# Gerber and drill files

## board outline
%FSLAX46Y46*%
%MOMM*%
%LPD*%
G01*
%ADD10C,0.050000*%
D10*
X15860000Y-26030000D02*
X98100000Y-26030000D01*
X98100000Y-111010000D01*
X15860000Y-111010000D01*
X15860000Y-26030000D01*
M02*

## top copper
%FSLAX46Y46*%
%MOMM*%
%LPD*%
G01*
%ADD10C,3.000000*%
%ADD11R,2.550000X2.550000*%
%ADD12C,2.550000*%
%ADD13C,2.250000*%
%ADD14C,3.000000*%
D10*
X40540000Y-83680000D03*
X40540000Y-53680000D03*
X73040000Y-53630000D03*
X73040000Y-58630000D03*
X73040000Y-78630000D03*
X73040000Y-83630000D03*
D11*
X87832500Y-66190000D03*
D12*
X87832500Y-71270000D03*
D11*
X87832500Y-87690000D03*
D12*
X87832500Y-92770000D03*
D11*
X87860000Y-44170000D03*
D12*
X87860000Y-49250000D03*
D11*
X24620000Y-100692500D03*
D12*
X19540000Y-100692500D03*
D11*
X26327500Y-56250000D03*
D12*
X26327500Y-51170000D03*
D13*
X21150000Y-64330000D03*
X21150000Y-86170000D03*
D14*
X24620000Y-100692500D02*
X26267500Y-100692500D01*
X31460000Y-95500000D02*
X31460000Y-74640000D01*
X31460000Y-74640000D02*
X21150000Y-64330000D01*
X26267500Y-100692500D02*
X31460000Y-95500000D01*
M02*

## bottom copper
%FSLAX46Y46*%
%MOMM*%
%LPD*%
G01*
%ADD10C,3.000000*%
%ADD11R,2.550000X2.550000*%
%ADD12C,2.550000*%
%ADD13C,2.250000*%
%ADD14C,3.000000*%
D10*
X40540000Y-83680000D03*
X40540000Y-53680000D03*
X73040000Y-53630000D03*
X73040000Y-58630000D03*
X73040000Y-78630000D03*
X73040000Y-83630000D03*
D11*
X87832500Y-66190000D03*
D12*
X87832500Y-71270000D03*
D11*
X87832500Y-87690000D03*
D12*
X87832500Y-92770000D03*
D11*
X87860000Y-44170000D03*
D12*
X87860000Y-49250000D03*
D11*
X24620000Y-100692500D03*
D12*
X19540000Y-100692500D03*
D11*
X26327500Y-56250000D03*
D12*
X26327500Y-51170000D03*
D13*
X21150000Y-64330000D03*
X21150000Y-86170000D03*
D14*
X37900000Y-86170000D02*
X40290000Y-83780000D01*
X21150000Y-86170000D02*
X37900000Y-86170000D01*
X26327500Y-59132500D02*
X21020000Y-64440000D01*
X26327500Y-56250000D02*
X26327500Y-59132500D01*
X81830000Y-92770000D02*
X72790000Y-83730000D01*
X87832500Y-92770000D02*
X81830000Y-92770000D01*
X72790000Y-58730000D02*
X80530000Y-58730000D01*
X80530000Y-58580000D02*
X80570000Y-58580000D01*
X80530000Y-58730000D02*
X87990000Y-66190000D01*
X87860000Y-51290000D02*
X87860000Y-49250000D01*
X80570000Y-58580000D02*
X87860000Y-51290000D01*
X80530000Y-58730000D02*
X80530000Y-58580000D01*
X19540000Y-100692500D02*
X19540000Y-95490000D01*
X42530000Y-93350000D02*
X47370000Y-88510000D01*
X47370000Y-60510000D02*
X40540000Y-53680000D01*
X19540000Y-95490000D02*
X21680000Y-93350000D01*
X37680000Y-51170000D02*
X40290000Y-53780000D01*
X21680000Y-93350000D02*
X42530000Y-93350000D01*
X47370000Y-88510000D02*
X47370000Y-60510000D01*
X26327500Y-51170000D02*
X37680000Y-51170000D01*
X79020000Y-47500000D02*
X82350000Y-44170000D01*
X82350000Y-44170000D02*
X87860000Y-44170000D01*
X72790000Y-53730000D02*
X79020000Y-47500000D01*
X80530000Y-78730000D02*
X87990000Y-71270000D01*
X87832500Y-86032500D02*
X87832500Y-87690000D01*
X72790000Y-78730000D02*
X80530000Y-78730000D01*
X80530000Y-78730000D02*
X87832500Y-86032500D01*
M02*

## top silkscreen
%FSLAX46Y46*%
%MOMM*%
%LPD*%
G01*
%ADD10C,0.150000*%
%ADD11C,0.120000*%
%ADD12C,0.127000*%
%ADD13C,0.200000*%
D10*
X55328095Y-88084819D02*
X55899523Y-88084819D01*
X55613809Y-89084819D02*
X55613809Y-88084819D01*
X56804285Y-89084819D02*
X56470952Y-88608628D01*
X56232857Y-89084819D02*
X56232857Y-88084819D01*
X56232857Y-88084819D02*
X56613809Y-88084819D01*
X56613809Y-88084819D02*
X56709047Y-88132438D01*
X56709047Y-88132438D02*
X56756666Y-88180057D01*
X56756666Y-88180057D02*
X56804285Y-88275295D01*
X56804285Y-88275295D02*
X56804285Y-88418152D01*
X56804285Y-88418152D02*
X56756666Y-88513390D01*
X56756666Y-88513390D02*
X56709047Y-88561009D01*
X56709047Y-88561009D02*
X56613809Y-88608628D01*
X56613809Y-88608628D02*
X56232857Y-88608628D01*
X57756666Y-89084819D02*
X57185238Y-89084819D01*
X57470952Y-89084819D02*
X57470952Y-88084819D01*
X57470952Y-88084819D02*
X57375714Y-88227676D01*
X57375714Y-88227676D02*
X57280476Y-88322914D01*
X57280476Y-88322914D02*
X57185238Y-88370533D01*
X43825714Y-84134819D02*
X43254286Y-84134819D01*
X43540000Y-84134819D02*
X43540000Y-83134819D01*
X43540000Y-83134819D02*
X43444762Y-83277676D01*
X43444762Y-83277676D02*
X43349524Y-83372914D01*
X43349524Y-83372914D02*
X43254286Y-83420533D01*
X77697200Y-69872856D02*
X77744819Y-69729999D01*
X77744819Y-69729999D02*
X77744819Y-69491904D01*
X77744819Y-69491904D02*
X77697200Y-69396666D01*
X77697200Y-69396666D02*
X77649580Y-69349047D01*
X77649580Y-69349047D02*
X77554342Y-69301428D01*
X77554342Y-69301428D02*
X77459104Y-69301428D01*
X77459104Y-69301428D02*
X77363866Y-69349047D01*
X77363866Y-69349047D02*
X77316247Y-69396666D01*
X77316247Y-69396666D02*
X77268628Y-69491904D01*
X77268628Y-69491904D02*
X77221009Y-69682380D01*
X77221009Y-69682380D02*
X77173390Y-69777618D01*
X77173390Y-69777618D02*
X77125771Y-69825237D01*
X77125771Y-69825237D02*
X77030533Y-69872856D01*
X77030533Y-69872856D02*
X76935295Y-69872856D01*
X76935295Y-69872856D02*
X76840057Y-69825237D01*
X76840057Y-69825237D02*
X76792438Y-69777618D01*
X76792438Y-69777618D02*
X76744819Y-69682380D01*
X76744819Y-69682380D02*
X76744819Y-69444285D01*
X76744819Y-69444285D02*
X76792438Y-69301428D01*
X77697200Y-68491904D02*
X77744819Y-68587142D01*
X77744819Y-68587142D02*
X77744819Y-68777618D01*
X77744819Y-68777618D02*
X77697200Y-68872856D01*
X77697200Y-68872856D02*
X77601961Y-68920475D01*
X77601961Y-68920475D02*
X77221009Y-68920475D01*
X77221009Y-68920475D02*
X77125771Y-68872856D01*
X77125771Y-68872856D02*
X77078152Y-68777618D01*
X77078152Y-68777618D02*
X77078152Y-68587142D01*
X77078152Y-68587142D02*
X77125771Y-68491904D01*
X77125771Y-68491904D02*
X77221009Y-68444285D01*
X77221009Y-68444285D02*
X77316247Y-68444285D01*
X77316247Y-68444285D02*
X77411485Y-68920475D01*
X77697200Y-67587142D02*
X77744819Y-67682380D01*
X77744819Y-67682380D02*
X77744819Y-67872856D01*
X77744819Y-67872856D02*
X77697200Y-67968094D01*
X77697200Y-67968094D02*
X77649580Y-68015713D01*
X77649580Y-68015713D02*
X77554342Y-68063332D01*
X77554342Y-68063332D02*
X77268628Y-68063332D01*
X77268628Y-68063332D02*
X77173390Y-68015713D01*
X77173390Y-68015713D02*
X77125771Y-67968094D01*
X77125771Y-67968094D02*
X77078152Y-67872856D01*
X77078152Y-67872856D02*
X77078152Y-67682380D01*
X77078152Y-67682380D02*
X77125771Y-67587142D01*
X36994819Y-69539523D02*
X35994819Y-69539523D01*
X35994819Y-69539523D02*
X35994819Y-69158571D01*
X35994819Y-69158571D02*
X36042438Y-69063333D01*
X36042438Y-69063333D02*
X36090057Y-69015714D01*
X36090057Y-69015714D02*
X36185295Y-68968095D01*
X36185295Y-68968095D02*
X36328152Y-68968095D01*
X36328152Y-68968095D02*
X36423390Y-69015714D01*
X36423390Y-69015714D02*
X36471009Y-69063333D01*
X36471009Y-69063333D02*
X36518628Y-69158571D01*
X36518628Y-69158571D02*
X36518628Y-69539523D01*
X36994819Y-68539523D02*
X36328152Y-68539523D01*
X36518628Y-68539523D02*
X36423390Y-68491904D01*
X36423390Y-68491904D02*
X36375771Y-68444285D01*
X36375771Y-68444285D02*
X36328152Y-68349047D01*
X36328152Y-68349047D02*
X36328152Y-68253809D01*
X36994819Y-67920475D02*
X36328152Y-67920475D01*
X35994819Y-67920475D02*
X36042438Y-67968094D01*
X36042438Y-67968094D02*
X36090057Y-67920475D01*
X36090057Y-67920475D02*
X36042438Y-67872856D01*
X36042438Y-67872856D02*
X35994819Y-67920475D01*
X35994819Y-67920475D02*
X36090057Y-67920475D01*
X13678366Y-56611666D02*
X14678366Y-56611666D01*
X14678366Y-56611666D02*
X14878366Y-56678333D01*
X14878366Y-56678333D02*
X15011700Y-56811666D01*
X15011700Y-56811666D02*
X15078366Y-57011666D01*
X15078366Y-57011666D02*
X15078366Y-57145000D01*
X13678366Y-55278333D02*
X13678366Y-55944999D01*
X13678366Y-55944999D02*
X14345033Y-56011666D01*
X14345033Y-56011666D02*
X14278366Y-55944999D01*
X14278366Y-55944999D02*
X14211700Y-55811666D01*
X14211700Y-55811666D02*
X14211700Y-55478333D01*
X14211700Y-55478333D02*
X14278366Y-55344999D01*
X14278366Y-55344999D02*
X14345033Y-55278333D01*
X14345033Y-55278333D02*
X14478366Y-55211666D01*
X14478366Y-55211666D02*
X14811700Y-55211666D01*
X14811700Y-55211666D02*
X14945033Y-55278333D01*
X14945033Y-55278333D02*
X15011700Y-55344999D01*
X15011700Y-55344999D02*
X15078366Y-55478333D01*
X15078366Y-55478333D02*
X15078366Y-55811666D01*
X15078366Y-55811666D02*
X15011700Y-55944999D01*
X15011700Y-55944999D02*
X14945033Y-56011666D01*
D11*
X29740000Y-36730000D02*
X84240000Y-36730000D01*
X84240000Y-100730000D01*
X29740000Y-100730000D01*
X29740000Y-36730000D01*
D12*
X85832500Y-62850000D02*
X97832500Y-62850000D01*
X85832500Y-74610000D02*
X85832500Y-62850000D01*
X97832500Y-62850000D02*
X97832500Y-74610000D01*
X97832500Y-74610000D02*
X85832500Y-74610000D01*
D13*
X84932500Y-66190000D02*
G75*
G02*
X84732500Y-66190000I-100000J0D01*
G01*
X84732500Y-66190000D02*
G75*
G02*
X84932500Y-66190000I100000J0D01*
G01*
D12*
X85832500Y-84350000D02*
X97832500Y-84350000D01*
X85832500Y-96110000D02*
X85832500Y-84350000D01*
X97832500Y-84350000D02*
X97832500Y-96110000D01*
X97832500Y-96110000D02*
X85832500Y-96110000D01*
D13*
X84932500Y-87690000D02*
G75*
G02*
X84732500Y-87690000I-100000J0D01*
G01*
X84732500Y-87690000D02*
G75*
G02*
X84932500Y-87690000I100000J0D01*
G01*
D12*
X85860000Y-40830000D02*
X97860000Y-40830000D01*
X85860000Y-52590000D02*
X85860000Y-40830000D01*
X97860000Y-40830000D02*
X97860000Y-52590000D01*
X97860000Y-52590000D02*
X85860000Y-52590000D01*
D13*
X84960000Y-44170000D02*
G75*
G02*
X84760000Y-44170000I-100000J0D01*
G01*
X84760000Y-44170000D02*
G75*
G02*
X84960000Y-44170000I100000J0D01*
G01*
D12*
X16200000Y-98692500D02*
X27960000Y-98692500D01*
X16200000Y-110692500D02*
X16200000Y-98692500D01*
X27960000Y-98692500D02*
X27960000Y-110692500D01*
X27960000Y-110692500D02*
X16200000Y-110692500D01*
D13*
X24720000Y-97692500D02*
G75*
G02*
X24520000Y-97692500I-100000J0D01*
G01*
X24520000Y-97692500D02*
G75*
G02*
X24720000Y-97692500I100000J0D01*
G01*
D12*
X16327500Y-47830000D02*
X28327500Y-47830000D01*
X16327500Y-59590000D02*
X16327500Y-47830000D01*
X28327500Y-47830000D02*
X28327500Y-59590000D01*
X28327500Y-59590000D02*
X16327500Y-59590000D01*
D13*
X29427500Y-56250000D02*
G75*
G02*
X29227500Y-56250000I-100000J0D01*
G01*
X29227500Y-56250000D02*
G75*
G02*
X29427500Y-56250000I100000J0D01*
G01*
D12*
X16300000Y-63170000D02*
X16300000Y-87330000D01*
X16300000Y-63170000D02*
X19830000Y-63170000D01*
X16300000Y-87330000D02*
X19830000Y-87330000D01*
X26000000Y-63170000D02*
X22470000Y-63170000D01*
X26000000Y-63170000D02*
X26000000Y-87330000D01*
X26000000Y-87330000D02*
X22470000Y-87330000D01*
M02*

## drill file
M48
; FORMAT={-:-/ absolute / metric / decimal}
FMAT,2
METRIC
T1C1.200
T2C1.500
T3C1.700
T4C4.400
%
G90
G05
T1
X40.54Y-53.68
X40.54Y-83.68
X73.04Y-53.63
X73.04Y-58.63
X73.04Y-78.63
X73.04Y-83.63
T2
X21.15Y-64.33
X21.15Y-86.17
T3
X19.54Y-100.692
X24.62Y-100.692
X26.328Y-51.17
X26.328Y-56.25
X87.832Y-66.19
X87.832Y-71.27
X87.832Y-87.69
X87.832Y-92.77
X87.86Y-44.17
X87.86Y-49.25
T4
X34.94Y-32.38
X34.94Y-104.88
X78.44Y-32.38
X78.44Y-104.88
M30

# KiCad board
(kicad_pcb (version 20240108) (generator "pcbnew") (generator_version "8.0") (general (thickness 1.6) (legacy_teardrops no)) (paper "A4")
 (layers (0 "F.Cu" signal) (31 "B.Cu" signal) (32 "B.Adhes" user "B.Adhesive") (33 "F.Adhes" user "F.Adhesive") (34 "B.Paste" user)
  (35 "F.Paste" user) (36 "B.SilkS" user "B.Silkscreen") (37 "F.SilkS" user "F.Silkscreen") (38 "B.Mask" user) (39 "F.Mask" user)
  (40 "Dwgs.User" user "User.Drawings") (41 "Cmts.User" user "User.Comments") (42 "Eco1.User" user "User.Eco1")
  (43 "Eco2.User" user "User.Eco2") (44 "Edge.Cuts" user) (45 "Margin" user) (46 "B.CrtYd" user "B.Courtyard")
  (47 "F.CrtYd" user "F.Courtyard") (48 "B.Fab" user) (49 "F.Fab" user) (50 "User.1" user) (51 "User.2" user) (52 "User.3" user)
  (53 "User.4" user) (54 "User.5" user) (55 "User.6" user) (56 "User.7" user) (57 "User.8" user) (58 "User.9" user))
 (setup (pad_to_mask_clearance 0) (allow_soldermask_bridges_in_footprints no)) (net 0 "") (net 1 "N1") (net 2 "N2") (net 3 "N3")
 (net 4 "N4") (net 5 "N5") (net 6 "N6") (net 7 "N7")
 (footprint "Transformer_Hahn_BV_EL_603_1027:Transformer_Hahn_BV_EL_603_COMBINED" (layer "F.Cu") (at 56.59 89.13)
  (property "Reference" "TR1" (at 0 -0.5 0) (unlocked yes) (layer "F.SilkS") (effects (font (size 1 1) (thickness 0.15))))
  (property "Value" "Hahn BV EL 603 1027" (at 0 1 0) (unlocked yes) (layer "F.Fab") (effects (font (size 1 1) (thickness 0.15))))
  (fp_rect (start -26.85 -52.4) (end 27.65 11.6) (stroke (width 0.12) (type default)) (fill none) (layer "F.SilkS"))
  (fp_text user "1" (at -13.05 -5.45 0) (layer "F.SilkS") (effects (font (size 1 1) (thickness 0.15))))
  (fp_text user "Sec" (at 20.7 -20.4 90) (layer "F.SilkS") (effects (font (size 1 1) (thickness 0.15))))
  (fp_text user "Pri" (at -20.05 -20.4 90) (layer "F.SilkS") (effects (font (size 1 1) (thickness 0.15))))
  (pad "" np_thru_hole circle (at -21.65 -56.75) (size 4.4 4.4) (drill 4.4) (layers "F&B.Cu" "*.Mask"))
  (pad "" np_thru_hole circle (at -21.65 15.75) (size 4.4 4.4) (drill 4.4) (layers "F&B.Cu" "*.Mask"))
  (pad "" np_thru_hole circle (at 21.85 -56.75) (size 4.4 4.4) (drill 4.4) (layers "F&B.Cu" "*.Mask"))
  (pad "" np_thru_hole circle (at 21.85 15.75) (size 4.4 4.4) (drill 4.4) (layers "F&B.Cu" "*.Mask"))
  (pad "1" thru_hole circle (at -16.05 -5.45) (size 3 3) (drill 1.2) (layers "*.Cu" "*.Mask") (remove_unused_layers no) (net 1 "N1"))
  (pad "7" thru_hole circle (at -16.05 -35.45) (size 3 3) (drill 1.2) (layers "*.Cu" "*.Mask") (remove_unused_layers no) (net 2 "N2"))
  (pad "8" thru_hole circle (at 16.45 -35.5) (size 3 3) (drill 1.2) (layers "*.Cu" "*.Mask") (remove_unused_layers no) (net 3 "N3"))
  (pad "9" thru_hole circle (at 16.45 -30.5) (size 3 3) (drill 1.2) (layers "*.Cu" "*.Mask") (remove_unused_layers no) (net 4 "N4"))
  (pad "13" thru_hole circle (at 16.45 -10.5) (size 3 3) (drill 1.2) (layers "*.Cu" "*.Mask") (remove_unused_layers no) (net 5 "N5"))
  (pad "14" thru_hole circle (at 16.45 -5.5) (size 3 3) (drill 1.2) (layers "*.Cu" "*.Mask") (remove_unused_layers no) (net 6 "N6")))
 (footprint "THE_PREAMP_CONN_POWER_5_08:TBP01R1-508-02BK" (layer "F.Cu") (at 87.8325 66.19 -90)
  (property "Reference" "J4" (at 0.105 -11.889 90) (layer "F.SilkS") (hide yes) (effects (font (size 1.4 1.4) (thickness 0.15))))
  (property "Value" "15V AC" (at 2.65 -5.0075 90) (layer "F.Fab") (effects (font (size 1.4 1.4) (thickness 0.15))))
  (fp_line (start -3.34 2) (end -3.34 -10) (stroke (width 0.127) (type solid)) (layer "F.SilkS"))
  (fp_line (start 8.42 2) (end -3.34 2) (stroke (width 0.127) (type solid)) (layer "F.SilkS"))
  (fp_line (start -3.34 -10) (end 8.42 -10) (stroke (width 0.127) (type solid)) (layer "F.SilkS"))
  (fp_line (start 8.42 -10) (end 8.42 2) (stroke (width 0.127) (type solid)) (layer "F.SilkS"))
  (fp_circle (center 0 3) (end 0.1 3) (stroke (width 0.2) (type solid)) (fill none) (layer "F.SilkS"))
  (pad "1" thru_hole rect (at 0 0 270) (size 2.55 2.55) (drill 1.7) (layers "*.Cu" "*.Mask") (remove_unused_layers no) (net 4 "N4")
   (solder_mask_margin 0.102))
  (pad "2" thru_hole circle (at 5.08 0 270) (size 2.55 2.55) (drill 1.7) (layers "*.Cu" "*.Mask") (remove_unused_layers no) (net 5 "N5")
   (solder_mask_margin 0.102)))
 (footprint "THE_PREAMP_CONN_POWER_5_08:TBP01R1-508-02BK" (layer "F.Cu") (at 87.8325 87.69 -90)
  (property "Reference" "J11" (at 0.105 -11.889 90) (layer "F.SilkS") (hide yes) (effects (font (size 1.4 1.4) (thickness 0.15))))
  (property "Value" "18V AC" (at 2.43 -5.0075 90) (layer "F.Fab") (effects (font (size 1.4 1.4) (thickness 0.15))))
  (fp_line (start -3.34 2) (end -3.34 -10) (stroke (width 0.127) (type solid)) (layer "F.SilkS"))
  (fp_line (start 8.42 2) (end -3.34 2) (stroke (width 0.127) (type solid)) (layer "F.SilkS"))
  (fp_line (start -3.34 -10) (end 8.42 -10) (stroke (width 0.127) (type solid)) (layer "F.SilkS"))
  (fp_line (start 8.42 -10) (end 8.42 2) (stroke (width 0.127) (type solid)) (layer "F.SilkS"))
  (fp_circle (center 0 3) (end 0.1 3) (stroke (width 0.2) (type solid)) (fill none) (layer "F.SilkS"))
  (pad "1" thru_hole rect (at 0 0 270) (size 2.55 2.55) (drill 1.7) (layers "*.Cu" "*.Mask") (remove_unused_layers no) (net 5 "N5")
   (solder_mask_margin 0.102))
  (pad "2" thru_hole circle (at 5.08 0 270) (size 2.55 2.55) (drill 1.7) (layers "*.Cu" "*.Mask") (remove_unused_layers no) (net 6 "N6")
   (solder_mask_margin 0.102)))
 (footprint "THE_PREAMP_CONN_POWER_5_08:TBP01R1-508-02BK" (layer "F.Cu") (at 87.86 44.17 -90)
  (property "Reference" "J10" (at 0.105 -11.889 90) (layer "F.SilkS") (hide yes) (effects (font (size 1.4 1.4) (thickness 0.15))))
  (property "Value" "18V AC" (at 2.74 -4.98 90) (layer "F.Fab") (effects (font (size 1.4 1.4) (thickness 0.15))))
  (fp_line (start -3.34 2) (end -3.34 -10) (stroke (width 0.127) (type solid)) (layer "F.SilkS"))
  (fp_line (start 8.42 2) (end -3.34 2) (stroke (width 0.127) (type solid)) (layer "F.SilkS"))
  (fp_line (start -3.34 -10) (end 8.42 -10) (stroke (width 0.127) (type solid)) (layer "F.SilkS"))
  (fp_line (start 8.42 -10) (end 8.42 2) (stroke (width 0.127) (type solid)) (layer "F.SilkS"))
  (fp_circle (center 0 3) (end 0.1 3) (stroke (width 0.2) (type solid)) (fill none) (layer "F.SilkS"))
  (pad "1" thru_hole rect (at 0 0 270) (size 2.55 2.55) (drill 1.7) (layers "*.Cu" "*.Mask") (remove_unused_layers no) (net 3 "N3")
   (solder_mask_margin 0.102))
  (pad "2" thru_hole circle (at 5.08 0 270) (size 2.55 2.55) (drill 1.7) (layers "*.Cu" "*.Mask") (remove_unused_layers no) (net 4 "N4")
   (solder_mask_margin 0.102)))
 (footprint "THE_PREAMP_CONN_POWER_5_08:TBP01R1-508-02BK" (layer "F.Cu") (at 24.62 100.6925 180)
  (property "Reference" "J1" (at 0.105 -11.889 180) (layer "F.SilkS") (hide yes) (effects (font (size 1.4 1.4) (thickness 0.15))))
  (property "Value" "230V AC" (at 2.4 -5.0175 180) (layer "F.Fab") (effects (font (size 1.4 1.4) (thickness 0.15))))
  (fp_line (start 8.42 2) (end -3.34 2) (stroke (width 0.127) (type solid)) (layer "F.SilkS"))
  (fp_line (start 8.42 -10) (end 8.42 2) (stroke (width 0.127) (type solid)) (layer "F.SilkS"))
  (fp_line (start -3.34 2) (end -3.34 -10) (stroke (width 0.127) (type solid)) (layer "F.SilkS"))
  (fp_line (start -3.34 -10) (end 8.42 -10) (stroke (width 0.127) (type solid)) (layer "F.SilkS"))
  (fp_circle (center 0 3) (end 0.1 3) (stroke (width 0.2) (type solid)) (fill none) (layer "F.SilkS"))
  (pad "1" thru_hole rect (at 0 0 180) (size 2.55 2.55) (drill 1.7) (layers "*.Cu" "*.Mask") (remove_unused_layers no) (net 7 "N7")
   (solder_mask_margin 0.102))
  (pad "2" thru_hole circle (at 5.08 0 180) (size 2.55 2.55) (drill 1.7) (layers "*.Cu" "*.Mask") (remove_unused_layers no) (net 2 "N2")
   (solder_mask_margin 0.102)))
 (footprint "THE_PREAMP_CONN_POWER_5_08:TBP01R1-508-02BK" (layer "F.Cu") (at 26.3275 56.25 90)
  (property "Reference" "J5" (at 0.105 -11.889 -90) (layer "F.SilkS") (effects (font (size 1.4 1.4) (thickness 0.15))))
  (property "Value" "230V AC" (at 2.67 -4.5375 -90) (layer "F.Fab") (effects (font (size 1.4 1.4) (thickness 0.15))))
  (fp_line (start 8.42 -10) (end 8.42 2) (stroke (width 0.127) (type solid)) (layer "F.SilkS"))
  (fp_line (start -3.34 -10) (end 8.42 -10) (stroke (width 0.127) (type solid)) (layer "F.SilkS"))
  (fp_line (start 8.42 2) (end -3.34 2) (stroke (width 0.127) (type solid)) (layer "F.SilkS"))
  (fp_line (start -3.34 2) (end -3.34 -10) (stroke (width 0.127) (type solid)) (layer "F.SilkS"))
  (fp_circle (center 0 3) (end 0.1 3) (stroke (width 0.2) (type solid)) (fill none) (layer "F.SilkS"))
  (pad "1" thru_hole rect (at 0 0 90) (size 2.55 2.55) (drill 1.7) (layers "*.Cu" "*.Mask") (remove_unused_layers no) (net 7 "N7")
   (solder_mask_margin 0.102))
  (pad "2" thru_hole circle (at 5.08 0 90) (size 2.55 2.55) (drill 1.7) (layers "*.Cu" "*.Mask") (remove_unused_layers no) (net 2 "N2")
   (solder_mask_margin 0.102)))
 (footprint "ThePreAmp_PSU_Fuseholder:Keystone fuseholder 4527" (layer "F.Cu") (at 21.15 75.25 -90)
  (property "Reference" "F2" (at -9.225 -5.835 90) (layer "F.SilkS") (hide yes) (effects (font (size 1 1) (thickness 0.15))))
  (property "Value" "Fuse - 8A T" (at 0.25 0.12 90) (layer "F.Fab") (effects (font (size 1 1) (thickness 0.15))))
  (fp_line (start -12.08 4.85) (end 12.08 4.85) (stroke (width 0.127) (type solid)) (layer "F.SilkS"))
  (fp_line (start -12.08 4.85) (end -12.08 1.32) (stroke (width 0.127) (type solid)) (layer "F.SilkS"))
  (fp_line (start 12.08 4.85) (end 12.08 1.32) (stroke (width 0.127) (type solid)) (layer "F.SilkS"))
  (fp_line (start -12.08 -4.85) (end -12.08 -1.32) (stroke (width 0.127) (type solid)) (layer "F.SilkS"))
  (fp_line (start -12.08 -4.85) (end 12.08 -4.85) (stroke (width 0.127) (type solid)) (layer "F.SilkS"))
  (fp_line (start 12.08 -4.85) (end 12.08 -1.32) (stroke (width 0.127) (type solid)) (layer "F.SilkS"))
  (pad "1" thru_hole circle (at -10.92 0 270) (size 2.25 2.25) (drill 1.5) (layers "*.Cu" "*.Mask") (remove_unused_layers no) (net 7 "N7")
   (solder_mask_margin 0.102))
  (pad "2" thru_hole circle (at 10.92 0 270) (size 2.25 2.25) (drill 1.5) (layers "*.Cu" "*.Mask") (remove_unused_layers no) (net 1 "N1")
   (solder_mask_margin 0.102)))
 (gr_rect (start 15.86 26.03) (end 98.1 111.01) (stroke (width 0.05) (type default)) (fill none) (layer "Edge.Cuts"))
 (segment (start 37.9 86.17) (end 40.29 83.78) (width 3) (layer "B.Cu") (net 1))
 (segment (start 21.15 86.17) (end 37.9 86.17) (width 3) (layer "B.Cu") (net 1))
 (segment (start 24.62 100.6925) (end 26.2675 100.6925) (width 3) (layer "F.Cu") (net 7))
 (segment (start 31.46 95.5) (end 31.46 74.64) (width 3) (layer "F.Cu") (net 7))
 (segment (start 31.46 74.64) (end 21.15 64.33) (width 3) (layer "F.Cu") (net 7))
 (segment (start 26.2675 100.6925) (end 31.46 95.5) (width 3) (layer "F.Cu") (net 7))
 (segment (start 26.3275 59.1325) (end 21.02 64.44) (width 3) (layer "B.Cu") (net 7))
 (segment (start 26.3275 56.25) (end 26.3275 59.1325) (width 3) (layer "B.Cu") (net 7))
 (segment (start 81.83 92.77) (end 72.79 83.73) (width 3) (layer "B.Cu") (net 6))
 (segment (start 87.8325 92.77) (end 81.83 92.77) (width 3) (layer "B.Cu") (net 6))
 (segment (start 72.79 58.73) (end 80.53 58.73) (width 3) (layer "B.Cu") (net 4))
 (segment (start 80.53 58.58) (end 80.57 58.58) (width 3) (layer "B.Cu") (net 4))
 (segment (start 80.53 58.73) (end 87.99 66.19) (width 3) (layer "B.Cu") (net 4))
 (segment (start 87.86 51.29) (end 87.86 49.25) (width 3) (layer "B.Cu") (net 4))
 (segment (start 80.57 58.58) (end 87.86 51.29) (width 3) (layer "B.Cu") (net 4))
 (segment (start 80.53 58.73) (end 80.53 58.58) (width 3) (layer "B.Cu") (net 4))
 (segment (start 19.54 100.6925) (end 19.54 95.49) (width 3) (layer "B.Cu") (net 2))
 (segment (start 42.53 93.35) (end 47.37 88.51) (width 3) (layer "B.Cu") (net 2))
 (segment (start 47.37 60.51) (end 40.54 53.68) (width 3) (layer "B.Cu") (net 2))
 (segment (start 19.54 95.49) (end 21.68 93.35) (width 3) (layer "B.Cu") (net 2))
 (segment (start 37.68 51.17) (end 40.29 53.78) (width 3) (layer "B.Cu") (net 2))
 (segment (start 21.68 93.35) (end 42.53 93.35) (width 3) (layer "B.Cu") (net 2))
 (segment (start 47.37 88.51) (end 47.37 60.51) (width 3) (layer "B.Cu") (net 2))
 (segment (start 26.3275 51.17) (end 37.68 51.17) (width 3) (layer "B.Cu") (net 2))
 (segment (start 79.02 47.5) (end 82.35 44.17) (width 3) (layer "B.Cu") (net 3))
 (segment (start 82.35 44.17) (end 87.86 44.17) (width 3) (layer "B.Cu") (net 3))
 (segment (start 72.79 53.73) (end 79.02 47.5) (width 3) (layer "B.Cu") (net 3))
 (segment (start 80.53 78.73) (end 87.99 71.27) (width 3) (layer "B.Cu") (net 5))
 (segment (start 87.8325 86.0325) (end 87.8325 87.69) (width 3) (layer "B.Cu") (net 5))
 (segment (start 72.79 78.73) (end 80.53 78.73) (width 3) (layer "B.Cu") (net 5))
 (segment (start 80.53 78.73) (end 87.8325 86.0325) (width 3) (layer "B.Cu") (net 5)))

